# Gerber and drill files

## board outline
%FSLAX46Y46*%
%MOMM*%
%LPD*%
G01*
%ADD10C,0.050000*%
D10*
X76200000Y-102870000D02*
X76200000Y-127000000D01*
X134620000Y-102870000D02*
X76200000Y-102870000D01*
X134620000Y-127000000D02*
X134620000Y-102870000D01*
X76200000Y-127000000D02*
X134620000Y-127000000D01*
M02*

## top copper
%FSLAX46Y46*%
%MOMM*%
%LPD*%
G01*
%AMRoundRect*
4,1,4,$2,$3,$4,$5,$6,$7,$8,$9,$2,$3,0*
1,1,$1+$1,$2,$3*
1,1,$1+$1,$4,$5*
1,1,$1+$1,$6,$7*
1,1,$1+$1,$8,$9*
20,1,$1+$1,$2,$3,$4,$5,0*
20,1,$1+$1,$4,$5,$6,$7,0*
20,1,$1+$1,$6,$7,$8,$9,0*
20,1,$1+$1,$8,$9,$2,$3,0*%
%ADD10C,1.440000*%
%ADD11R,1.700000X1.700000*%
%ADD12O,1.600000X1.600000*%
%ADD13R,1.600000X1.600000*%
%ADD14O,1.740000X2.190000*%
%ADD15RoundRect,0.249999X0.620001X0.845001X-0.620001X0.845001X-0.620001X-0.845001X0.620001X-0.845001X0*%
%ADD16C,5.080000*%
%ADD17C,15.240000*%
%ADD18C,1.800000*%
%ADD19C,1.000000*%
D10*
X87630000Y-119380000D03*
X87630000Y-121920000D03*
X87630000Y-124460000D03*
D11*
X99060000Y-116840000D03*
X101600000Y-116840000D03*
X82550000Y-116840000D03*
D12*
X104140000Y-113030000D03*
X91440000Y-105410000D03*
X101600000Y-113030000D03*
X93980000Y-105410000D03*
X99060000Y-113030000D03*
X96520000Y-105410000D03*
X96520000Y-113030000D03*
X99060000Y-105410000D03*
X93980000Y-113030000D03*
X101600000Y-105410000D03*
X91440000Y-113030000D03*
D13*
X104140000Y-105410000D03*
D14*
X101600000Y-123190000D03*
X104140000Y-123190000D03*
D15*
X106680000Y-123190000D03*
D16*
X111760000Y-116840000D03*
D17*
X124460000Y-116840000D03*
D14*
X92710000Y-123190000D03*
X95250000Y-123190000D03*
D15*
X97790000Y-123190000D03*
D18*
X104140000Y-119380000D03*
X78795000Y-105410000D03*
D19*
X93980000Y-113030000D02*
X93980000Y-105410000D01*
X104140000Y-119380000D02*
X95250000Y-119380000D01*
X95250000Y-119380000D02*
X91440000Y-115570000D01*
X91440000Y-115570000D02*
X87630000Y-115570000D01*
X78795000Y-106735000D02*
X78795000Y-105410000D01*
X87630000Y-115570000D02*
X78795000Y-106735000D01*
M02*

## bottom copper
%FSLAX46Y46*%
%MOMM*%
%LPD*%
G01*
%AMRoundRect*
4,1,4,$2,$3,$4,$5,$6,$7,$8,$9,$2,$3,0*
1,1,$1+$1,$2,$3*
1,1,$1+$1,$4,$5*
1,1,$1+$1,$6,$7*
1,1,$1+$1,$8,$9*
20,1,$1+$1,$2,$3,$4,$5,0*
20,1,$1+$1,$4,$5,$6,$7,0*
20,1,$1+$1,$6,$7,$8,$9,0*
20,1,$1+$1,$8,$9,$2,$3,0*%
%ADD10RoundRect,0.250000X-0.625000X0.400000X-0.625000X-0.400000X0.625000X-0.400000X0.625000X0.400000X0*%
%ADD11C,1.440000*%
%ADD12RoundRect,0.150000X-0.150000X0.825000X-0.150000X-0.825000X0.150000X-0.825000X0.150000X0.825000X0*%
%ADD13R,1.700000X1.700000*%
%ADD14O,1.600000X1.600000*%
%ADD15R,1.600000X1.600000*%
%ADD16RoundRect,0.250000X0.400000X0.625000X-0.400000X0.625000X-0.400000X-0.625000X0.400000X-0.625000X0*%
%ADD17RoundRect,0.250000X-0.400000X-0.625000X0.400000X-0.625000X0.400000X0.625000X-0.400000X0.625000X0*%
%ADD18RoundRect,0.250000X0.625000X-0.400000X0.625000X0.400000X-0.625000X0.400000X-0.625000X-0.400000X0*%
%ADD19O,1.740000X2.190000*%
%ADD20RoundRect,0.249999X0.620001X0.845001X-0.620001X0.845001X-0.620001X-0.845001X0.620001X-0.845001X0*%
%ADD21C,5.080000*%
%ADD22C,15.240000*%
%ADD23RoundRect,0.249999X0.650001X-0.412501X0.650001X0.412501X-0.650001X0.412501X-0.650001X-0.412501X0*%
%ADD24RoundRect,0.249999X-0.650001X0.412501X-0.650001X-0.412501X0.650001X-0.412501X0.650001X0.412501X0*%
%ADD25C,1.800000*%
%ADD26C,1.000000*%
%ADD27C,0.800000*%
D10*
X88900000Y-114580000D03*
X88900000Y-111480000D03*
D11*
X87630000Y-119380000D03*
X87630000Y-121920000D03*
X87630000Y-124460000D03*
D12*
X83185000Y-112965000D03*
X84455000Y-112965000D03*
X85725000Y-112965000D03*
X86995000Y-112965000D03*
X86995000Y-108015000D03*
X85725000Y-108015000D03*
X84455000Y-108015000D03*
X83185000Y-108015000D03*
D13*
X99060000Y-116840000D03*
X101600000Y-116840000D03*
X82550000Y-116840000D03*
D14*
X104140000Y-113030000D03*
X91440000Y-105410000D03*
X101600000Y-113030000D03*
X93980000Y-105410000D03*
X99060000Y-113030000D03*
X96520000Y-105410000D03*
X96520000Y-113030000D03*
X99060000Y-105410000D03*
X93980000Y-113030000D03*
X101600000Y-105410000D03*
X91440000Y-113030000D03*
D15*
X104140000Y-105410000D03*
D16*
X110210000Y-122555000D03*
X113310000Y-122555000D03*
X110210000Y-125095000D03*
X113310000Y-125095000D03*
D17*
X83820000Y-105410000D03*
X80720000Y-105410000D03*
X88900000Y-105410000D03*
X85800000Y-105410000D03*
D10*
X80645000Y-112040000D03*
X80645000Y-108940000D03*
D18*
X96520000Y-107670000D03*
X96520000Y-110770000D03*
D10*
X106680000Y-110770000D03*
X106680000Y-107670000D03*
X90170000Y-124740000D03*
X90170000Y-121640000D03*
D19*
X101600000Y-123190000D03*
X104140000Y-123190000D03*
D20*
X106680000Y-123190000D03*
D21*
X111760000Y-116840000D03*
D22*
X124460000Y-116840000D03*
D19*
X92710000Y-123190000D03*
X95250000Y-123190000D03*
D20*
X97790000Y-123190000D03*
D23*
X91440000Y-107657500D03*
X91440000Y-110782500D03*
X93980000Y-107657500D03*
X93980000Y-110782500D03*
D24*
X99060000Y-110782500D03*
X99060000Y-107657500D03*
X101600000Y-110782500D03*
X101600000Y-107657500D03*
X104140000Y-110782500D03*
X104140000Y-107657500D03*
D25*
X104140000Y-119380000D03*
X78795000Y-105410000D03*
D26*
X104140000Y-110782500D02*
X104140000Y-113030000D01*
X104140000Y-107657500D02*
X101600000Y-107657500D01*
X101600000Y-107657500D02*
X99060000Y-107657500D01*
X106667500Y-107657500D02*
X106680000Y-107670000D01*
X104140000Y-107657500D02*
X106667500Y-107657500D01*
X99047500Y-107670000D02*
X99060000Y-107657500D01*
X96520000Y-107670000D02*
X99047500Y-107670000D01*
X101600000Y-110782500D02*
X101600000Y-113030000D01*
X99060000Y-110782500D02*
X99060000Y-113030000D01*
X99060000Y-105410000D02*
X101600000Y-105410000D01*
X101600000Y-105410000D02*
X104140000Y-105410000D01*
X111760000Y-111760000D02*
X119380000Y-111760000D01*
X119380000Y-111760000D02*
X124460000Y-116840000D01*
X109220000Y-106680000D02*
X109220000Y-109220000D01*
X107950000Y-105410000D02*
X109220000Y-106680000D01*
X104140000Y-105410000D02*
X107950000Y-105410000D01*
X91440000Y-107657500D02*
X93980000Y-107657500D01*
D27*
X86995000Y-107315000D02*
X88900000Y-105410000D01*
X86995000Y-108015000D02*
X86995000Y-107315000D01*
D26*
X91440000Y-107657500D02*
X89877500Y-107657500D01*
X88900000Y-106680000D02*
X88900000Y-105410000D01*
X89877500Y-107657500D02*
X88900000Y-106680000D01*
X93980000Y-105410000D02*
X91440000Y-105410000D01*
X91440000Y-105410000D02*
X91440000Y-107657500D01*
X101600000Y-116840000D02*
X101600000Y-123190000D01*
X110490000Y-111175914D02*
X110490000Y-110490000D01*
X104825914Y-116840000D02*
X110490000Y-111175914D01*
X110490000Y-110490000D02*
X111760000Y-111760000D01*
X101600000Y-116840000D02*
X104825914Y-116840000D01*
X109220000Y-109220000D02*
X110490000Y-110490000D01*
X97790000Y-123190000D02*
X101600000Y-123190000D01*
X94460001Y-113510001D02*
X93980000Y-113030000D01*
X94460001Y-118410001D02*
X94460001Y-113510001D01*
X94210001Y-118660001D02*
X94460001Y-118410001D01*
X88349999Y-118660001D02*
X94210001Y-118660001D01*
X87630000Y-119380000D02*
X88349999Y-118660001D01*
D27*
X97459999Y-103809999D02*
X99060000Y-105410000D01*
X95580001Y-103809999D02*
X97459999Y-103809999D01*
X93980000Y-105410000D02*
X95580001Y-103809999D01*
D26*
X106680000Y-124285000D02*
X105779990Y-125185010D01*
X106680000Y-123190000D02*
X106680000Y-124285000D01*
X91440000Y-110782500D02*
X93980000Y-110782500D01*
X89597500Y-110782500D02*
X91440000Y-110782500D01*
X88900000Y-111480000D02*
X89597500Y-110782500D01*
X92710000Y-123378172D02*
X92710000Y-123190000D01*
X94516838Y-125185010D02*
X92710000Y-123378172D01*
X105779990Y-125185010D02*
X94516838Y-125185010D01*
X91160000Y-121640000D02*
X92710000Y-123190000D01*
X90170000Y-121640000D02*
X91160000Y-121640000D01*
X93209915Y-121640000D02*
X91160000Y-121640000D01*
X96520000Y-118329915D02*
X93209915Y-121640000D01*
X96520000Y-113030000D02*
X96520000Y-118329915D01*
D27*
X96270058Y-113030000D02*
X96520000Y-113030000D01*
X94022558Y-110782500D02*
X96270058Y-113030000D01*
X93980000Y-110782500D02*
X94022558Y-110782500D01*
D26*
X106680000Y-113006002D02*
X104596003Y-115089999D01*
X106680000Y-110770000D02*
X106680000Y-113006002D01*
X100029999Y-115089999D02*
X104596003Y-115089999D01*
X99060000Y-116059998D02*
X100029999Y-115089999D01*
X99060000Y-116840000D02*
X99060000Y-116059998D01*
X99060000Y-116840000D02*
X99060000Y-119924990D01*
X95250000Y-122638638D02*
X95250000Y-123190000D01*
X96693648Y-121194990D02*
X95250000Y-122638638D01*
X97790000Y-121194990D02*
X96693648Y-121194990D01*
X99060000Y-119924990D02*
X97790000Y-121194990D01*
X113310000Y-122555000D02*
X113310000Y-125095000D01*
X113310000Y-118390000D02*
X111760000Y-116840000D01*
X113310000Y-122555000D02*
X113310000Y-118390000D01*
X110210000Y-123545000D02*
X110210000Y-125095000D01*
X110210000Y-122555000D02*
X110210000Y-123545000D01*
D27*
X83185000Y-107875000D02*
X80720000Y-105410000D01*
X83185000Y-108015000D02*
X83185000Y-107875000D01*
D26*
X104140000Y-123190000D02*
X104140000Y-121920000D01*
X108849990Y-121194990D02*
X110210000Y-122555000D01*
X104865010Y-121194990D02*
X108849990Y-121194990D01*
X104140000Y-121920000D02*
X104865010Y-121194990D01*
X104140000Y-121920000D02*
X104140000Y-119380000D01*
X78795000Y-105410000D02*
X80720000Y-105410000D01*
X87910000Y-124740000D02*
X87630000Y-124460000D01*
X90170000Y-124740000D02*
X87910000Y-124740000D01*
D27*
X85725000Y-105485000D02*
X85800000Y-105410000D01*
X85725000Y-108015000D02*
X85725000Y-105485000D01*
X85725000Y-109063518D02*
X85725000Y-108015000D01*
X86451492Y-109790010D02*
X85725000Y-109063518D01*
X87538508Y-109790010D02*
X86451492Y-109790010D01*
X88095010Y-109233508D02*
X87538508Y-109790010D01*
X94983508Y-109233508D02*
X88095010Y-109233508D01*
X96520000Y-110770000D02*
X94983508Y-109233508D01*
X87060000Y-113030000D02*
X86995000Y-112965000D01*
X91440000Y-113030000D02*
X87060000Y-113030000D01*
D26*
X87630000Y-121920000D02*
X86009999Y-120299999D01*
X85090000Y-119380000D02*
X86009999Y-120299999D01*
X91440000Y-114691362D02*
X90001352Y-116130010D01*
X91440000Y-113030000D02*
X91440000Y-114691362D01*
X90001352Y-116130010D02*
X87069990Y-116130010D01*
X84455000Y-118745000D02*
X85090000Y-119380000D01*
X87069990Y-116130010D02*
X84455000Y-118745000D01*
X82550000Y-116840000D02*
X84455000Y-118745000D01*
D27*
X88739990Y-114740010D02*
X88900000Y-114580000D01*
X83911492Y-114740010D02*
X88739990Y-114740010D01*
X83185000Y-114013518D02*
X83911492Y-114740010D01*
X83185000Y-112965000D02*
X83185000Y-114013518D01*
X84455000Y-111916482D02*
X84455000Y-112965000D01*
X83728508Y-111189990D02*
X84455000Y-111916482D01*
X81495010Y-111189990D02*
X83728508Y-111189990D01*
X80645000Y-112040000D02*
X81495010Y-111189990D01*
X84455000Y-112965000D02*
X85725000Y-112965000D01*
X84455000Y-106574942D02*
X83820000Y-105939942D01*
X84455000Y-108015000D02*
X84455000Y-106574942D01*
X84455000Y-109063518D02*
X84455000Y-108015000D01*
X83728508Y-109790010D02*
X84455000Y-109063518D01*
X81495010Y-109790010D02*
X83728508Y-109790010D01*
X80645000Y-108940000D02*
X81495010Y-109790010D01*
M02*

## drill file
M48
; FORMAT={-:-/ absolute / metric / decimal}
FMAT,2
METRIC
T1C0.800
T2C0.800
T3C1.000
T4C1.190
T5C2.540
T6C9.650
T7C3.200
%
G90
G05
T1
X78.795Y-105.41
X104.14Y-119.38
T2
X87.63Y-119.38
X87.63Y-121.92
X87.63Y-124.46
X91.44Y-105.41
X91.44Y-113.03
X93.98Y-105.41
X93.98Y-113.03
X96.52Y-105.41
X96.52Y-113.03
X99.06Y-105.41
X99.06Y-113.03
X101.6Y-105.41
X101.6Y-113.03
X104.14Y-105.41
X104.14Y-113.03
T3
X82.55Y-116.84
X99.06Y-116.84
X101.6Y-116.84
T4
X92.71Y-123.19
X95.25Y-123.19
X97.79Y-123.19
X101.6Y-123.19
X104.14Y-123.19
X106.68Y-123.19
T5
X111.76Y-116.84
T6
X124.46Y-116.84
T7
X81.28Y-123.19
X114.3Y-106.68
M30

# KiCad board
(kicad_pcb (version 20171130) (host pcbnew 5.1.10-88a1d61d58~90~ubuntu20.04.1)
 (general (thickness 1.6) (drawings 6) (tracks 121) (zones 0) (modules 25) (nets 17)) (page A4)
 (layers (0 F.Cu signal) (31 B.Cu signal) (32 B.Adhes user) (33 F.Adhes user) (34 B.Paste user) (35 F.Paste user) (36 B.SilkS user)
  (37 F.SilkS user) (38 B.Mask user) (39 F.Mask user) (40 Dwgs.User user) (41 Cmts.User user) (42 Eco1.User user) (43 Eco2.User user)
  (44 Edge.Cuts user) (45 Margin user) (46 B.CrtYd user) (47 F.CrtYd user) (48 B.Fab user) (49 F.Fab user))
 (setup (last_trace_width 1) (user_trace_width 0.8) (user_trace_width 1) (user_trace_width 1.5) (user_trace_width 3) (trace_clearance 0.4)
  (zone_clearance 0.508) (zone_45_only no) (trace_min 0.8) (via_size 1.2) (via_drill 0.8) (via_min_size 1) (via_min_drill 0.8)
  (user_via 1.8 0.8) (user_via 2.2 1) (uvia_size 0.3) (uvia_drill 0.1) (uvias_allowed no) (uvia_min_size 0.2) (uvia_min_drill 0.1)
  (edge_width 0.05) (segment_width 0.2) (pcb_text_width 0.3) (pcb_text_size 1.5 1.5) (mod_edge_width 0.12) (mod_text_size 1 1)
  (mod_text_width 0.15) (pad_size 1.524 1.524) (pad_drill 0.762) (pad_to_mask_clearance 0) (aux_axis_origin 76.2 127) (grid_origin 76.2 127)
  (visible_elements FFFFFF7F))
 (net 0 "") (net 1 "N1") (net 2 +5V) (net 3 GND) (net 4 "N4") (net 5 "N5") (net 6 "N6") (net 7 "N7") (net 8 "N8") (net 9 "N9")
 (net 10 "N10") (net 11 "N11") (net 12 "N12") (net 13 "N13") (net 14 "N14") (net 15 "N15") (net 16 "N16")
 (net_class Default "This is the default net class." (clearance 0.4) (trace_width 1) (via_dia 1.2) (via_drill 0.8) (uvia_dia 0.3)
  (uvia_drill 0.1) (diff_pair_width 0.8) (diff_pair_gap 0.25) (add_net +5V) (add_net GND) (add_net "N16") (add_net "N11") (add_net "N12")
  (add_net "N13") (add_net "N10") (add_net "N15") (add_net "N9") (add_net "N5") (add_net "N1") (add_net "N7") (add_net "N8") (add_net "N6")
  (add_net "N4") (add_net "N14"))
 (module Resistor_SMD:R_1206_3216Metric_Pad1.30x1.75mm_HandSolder (layer B.Cu) (at 88.9 113.03 270)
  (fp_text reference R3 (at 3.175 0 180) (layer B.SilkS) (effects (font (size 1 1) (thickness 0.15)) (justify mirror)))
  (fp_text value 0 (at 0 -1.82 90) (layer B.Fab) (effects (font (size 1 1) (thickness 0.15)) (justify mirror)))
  (pad 2 smd roundrect (at 1.55 0 270) (size 1.3 1.75) (layers B.Cu B.Paste B.Mask) (roundrect_rratio 0.1923076923076923) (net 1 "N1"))
  (pad 1 smd roundrect (at -1.55 0 270) (size 1.3 1.75) (layers B.Cu B.Paste B.Mask) (roundrect_rratio 0.1923076923076923) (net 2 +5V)))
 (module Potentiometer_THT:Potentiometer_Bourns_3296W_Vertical (layer F.Cu) (at 87.63 124.46 270)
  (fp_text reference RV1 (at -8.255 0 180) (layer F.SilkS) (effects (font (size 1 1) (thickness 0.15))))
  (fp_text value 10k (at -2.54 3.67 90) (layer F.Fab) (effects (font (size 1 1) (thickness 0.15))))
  (pad 3 thru_hole circle (at -5.08 0 270) (size 1.44 1.44) (drill 0.8) (layers *.Cu *.Mask) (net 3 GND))
  (pad 2 thru_hole circle (at -2.54 0 270) (size 1.44 1.44) (drill 0.8) (layers *.Cu *.Mask) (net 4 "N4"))
  (pad 1 thru_hole circle (at 0 0 270) (size 1.44 1.44) (drill 0.8) (layers *.Cu *.Mask) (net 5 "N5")))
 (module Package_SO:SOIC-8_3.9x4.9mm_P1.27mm (layer B.Cu) (at 85.09 110.49 270)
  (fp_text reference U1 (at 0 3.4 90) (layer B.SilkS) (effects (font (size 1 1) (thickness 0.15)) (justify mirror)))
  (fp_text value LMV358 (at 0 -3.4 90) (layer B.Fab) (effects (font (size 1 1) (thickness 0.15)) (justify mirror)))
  (pad 8 smd roundrect (at 2.475 1.905 270) (size 1.95 0.6) (layers B.Cu B.Paste B.Mask) (roundrect_rratio 0.25) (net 1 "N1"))
  (pad 7 smd roundrect (at 2.475 0.635 270) (size 1.95 0.6) (layers B.Cu B.Paste B.Mask) (roundrect_rratio 0.25) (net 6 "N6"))
  (pad 6 smd roundrect (at 2.475 -0.635 270) (size 1.95 0.6) (layers B.Cu B.Paste B.Mask) (roundrect_rratio 0.25) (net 6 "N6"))
  (pad 5 smd roundrect (at 2.475 -1.905 270) (size 1.95 0.6) (layers B.Cu B.Paste B.Mask) (roundrect_rratio 0.25) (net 4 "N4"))
  (pad 4 smd roundrect (at -2.475 -1.905 270) (size 1.95 0.6) (layers B.Cu B.Paste B.Mask) (roundrect_rratio 0.25) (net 3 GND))
  (pad 3 smd roundrect (at -2.475 -0.635 270) (size 1.95 0.6) (layers B.Cu B.Paste B.Mask) (roundrect_rratio 0.25) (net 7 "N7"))
  (pad 2 smd roundrect (at -2.475 0.635 270) (size 1.95 0.6) (layers B.Cu B.Paste B.Mask) (roundrect_rratio 0.25) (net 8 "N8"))
  (pad 1 smd roundrect (at -2.475 1.905 270) (size 1.95 0.6) (layers B.Cu B.Paste B.Mask) (roundrect_rratio 0.25) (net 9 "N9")))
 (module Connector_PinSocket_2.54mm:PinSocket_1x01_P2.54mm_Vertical (layer F.Cu) (at 99.06 116.84)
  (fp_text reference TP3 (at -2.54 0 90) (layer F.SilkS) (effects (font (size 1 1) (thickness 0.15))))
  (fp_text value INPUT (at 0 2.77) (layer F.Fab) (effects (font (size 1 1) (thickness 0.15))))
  (pad 1 thru_hole rect (at 0 0) (size 1.7 1.7) (drill 1) (layers *.Cu *.Mask) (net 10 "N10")))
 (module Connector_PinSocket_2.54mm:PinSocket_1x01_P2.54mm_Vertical (layer F.Cu) (at 101.6 116.84)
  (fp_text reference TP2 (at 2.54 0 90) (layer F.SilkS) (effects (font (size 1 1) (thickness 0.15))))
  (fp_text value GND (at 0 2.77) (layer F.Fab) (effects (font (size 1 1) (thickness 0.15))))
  (pad 1 thru_hole rect (at 0 0) (size 1.7 1.7) (drill 1) (layers *.Cu *.Mask) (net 3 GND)))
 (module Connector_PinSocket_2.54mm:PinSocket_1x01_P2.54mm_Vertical (layer F.Cu) (at 82.55 116.84)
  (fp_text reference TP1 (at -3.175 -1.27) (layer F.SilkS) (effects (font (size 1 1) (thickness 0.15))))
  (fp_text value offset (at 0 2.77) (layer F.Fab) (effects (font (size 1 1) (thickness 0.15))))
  (pad 1 thru_hole rect (at 0 0) (size 1.7 1.7) (drill 1) (layers *.Cu *.Mask) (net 4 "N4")))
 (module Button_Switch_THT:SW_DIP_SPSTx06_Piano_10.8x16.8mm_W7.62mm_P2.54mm (layer F.Cu) (at 104.14 105.41 270)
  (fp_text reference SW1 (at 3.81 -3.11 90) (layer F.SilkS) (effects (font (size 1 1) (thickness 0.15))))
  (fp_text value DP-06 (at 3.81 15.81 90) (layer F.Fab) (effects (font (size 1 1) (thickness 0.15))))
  (pad 12 thru_hole oval (at 7.62 0 270) (size 1.6 1.6) (drill 0.8) (layers *.Cu *.Mask) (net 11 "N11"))
  (pad 6 thru_hole oval (at 0 12.7 270) (size 1.6 1.6) (drill 0.8) (layers *.Cu *.Mask) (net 3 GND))
  (pad 11 thru_hole oval (at 7.62 2.54 270) (size 1.6 1.6) (drill 0.8) (layers *.Cu *.Mask) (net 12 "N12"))
  (pad 5 thru_hole oval (at 0 10.16 270) (size 1.6 1.6) (drill 0.8) (layers *.Cu *.Mask) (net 3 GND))
  (pad 10 thru_hole oval (at 7.62 5.08 270) (size 1.6 1.6) (drill 0.8) (layers *.Cu *.Mask) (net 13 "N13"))
  (pad 4 thru_hole oval (at 0 7.62 270) (size 1.6 1.6) (drill 0.8) (layers *.Cu *.Mask) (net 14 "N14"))
  (pad 9 thru_hole oval (at 7.62 7.62 270) (size 1.6 1.6) (drill 0.8) (layers *.Cu *.Mask) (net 2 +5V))
  (pad 3 thru_hole oval (at 0 5.08 270) (size 1.6 1.6) (drill 0.8) (layers *.Cu *.Mask) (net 3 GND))
  (pad 8 thru_hole oval (at 7.62 10.16 270) (size 1.6 1.6) (drill 0.8) (layers *.Cu *.Mask) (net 3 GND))
  (pad 2 thru_hole oval (at 0 2.54 270) (size 1.6 1.6) (drill 0.8) (layers *.Cu *.Mask) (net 3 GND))
  (pad 7 thru_hole oval (at 7.62 12.7 270) (size 1.6 1.6) (drill 0.8) (layers *.Cu *.Mask) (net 4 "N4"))
  (pad 1 thru_hole rect (at 0 0 270) (size 1.6 1.6) (drill 0.8) (layers *.Cu *.Mask) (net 3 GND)))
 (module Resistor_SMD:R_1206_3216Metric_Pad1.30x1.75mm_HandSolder (layer B.Cu) (at 111.76 122.555 180)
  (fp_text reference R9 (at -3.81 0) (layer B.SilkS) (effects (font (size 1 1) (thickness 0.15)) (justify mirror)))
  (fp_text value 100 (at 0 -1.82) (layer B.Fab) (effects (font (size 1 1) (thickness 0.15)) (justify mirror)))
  (pad 2 smd roundrect (at 1.55 0 180) (size 1.3 1.75) (layers B.Cu B.Paste B.Mask) (roundrect_rratio 0.1923076923076923) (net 9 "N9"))
  (pad 1 smd roundrect (at -1.55 0 180) (size 1.3 1.75) (layers B.Cu B.Paste B.Mask) (roundrect_rratio 0.1923076923076923) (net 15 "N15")))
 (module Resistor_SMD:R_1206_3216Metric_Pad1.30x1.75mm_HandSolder (layer B.Cu) (at 111.76 125.095 180)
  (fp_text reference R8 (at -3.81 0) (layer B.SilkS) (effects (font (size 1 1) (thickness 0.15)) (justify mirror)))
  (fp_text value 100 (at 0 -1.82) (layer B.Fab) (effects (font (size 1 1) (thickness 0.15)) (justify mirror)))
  (pad 2 smd roundrect (at 1.55 0 180) (size 1.3 1.75) (layers B.Cu B.Paste B.Mask) (roundrect_rratio 0.1923076923076923) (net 9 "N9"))
  (pad 1 smd roundrect (at -1.55 0 180) (size 1.3 1.75) (layers B.Cu B.Paste B.Mask) (roundrect_rratio 0.1923076923076923) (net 15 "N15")))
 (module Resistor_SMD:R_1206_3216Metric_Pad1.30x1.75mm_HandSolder (layer B.Cu) (at 82.27 105.41)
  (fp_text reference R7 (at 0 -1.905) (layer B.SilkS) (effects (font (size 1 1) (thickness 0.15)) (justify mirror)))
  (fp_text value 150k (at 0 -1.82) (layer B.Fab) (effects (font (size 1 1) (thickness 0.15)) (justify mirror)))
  (pad 2 smd roundrect (at 1.55 0) (size 1.3 1.75) (layers B.Cu B.Paste B.Mask) (roundrect_rratio 0.1923076923076923) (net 8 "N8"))
  (pad 1 smd roundrect (at -1.55 0) (size 1.3 1.75) (layers B.Cu B.Paste B.Mask) (roundrect_rratio 0.1923076923076923) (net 9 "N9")))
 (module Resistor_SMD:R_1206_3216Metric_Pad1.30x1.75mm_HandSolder (layer B.Cu) (at 87.35 105.41)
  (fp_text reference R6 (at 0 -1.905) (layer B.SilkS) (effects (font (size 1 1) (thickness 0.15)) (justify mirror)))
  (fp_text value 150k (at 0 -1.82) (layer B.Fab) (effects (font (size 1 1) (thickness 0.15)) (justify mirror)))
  (pad 2 smd roundrect (at 1.55 0) (size 1.3 1.75) (layers B.Cu B.Paste B.Mask) (roundrect_rratio 0.1923076923076923) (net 3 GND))
  (pad 1 smd roundrect (at -1.55 0) (size 1.3 1.75) (layers B.Cu B.Paste B.Mask) (roundrect_rratio 0.1923076923076923) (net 7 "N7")))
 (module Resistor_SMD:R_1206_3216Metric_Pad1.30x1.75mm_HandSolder (layer B.Cu) (at 80.645 110.49 270)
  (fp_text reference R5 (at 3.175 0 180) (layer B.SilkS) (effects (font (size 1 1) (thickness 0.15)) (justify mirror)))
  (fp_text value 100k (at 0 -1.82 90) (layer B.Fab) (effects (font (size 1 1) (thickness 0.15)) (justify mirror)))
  (pad 2 smd roundrect (at 1.55 0 270) (size 1.3 1.75) (layers B.Cu B.Paste B.Mask) (roundrect_rratio 0.1923076923076923) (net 6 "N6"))
  (pad 1 smd roundrect (at -1.55 0 270) (size 1.3 1.75) (layers B.Cu B.Paste B.Mask) (roundrect_rratio 0.1923076923076923) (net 8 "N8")))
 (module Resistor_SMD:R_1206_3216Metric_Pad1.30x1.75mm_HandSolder (layer B.Cu) (at 96.52 109.22 90)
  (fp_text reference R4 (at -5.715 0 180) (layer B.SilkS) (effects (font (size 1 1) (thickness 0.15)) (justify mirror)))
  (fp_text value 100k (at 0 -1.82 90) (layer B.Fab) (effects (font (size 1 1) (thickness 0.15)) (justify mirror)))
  (pad 2 smd roundrect (at 1.55 0 90) (size 1.3 1.75) (layers B.Cu B.Paste B.Mask) (roundrect_rratio 0.1923076923076923) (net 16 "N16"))
  (pad 1 smd roundrect (at -1.55 0 90) (size 1.3 1.75) (layers B.Cu B.Paste B.Mask) (roundrect_rratio 0.1923076923076923) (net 7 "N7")))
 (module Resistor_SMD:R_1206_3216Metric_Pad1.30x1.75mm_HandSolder (layer B.Cu) (at 106.68 109.22 270)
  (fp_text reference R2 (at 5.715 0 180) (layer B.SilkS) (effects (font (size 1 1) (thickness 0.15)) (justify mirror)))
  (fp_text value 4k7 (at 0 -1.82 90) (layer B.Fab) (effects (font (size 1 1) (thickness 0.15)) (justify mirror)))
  (pad 2 smd roundrect (at 1.55 0 270) (size 1.3 1.75) (layers B.Cu B.Paste B.Mask) (roundrect_rratio 0.1923076923076923) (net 10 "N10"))
  (pad 1 smd roundrect (at -1.55 0 270) (size 1.3 1.75) (layers B.Cu B.Paste B.Mask) (roundrect_rratio 0.1923076923076923) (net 16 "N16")))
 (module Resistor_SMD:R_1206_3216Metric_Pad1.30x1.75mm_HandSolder (layer B.Cu) (at 90.17 123.19 270)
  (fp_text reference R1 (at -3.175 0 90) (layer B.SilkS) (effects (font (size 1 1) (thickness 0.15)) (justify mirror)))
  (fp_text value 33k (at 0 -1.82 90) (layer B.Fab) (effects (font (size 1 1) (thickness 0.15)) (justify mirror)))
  (pad 2 smd roundrect (at 1.55 0 270) (size 1.3 1.75) (layers B.Cu B.Paste B.Mask) (roundrect_rratio 0.1923076923076923) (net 5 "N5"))
  (pad 1 smd roundrect (at -1.55 0 270) (size 1.3 1.75) (layers B.Cu B.Paste B.Mask) (roundrect_rratio 0.1923076923076923) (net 2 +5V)))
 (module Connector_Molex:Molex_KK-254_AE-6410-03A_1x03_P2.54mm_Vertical (layer F.Cu) (at 106.68 123.19 180)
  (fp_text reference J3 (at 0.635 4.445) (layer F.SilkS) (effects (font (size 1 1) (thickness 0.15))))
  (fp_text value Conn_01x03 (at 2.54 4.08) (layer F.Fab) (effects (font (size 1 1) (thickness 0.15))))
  (pad 3 thru_hole oval (at 5.08 0 180) (size 1.74 2.19) (drill 1.19) (layers *.Cu *.Mask) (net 3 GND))
  (pad 2 thru_hole oval (at 2.54 0 180) (size 1.74 2.19) (drill 1.19) (layers *.Cu *.Mask) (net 9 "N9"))
  (pad 1 thru_hole roundrect (at 0 0 180) (size 1.74 2.19) (drill 1.19) (layers *.Cu *.Mask) (roundrect_rratio 0.1436775862068966)
   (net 2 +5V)))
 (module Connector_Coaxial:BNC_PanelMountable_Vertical (layer F.Cu) (at 111.76 116.84 180)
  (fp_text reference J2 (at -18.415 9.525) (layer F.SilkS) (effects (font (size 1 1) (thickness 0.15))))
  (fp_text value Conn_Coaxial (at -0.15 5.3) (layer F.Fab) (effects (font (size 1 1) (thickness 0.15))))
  (pad 1 thru_hole circle (at 0 0 180) (size 5.08 5.08) (drill 2.54) (layers *.Cu *.Mask) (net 15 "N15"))
  (pad 2 thru_hole circle (at -12.7 0 180) (size 15.24 15.24) (drill 9.65) (layers *.Cu *.Mask) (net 3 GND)))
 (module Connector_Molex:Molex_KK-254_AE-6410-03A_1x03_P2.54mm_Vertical (layer F.Cu) (at 97.79 123.19 180)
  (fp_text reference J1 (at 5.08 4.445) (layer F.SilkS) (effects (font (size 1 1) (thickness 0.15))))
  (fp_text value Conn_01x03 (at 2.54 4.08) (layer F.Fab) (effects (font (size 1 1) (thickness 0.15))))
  (pad 3 thru_hole oval (at 5.08 0 180) (size 1.74 2.19) (drill 1.19) (layers *.Cu *.Mask) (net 2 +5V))
  (pad 2 thru_hole oval (at 2.54 0 180) (size 1.74 2.19) (drill 1.19) (layers *.Cu *.Mask) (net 10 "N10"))
  (pad 1 thru_hole roundrect (at 0 0 180) (size 1.74 2.19) (drill 1.19) (layers *.Cu *.Mask) (roundrect_rratio 0.1436775862068966)
   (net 3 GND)))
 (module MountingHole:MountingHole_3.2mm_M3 (layer F.Cu) (at 114.3 106.68)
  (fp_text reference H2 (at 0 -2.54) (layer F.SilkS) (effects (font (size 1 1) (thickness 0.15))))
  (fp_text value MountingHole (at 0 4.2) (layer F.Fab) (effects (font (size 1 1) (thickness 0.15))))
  (pad 1 np_thru_hole circle (at 0 0) (size 3.2 3.2) (drill 3.2) (layers *.Cu *.Mask)))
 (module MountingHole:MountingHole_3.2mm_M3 (layer F.Cu) (at 81.28 123.19)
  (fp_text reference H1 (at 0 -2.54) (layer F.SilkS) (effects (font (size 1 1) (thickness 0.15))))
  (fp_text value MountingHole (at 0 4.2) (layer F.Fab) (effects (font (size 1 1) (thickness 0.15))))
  (pad 1 np_thru_hole circle (at 0 0) (size 3.2 3.2) (drill 3.2) (layers *.Cu *.Mask)))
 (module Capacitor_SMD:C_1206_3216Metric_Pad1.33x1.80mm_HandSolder (layer B.Cu) (at 91.44 109.22 90)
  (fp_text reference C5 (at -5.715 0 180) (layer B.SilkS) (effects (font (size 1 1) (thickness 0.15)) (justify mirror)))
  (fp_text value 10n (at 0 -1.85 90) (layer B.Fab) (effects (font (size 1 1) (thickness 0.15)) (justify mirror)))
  (pad 2 smd roundrect (at 1.5625 0 90) (size 1.325 1.8) (layers B.Cu B.Paste B.Mask) (roundrect_rratio 0.1886784905660377) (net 3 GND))
  (pad 1 smd roundrect (at -1.5625 0 90) (size 1.325 1.8) (layers B.Cu B.Paste B.Mask) (roundrect_rratio 0.1886784905660377) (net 2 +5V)))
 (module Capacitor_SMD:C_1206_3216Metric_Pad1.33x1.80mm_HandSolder (layer B.Cu) (at 93.98 109.22 90)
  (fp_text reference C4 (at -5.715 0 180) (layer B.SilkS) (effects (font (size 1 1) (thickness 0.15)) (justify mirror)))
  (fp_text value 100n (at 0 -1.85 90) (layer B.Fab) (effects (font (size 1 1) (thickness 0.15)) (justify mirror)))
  (pad 2 smd roundrect (at 1.5625 0 90) (size 1.325 1.8) (layers B.Cu B.Paste B.Mask) (roundrect_rratio 0.1886784905660377) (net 3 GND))
  (pad 1 smd roundrect (at -1.5625 0 90) (size 1.325 1.8) (layers B.Cu B.Paste B.Mask) (roundrect_rratio 0.1886784905660377) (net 2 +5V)))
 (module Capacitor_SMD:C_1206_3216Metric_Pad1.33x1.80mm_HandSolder (layer B.Cu) (at 99.06 109.22 270)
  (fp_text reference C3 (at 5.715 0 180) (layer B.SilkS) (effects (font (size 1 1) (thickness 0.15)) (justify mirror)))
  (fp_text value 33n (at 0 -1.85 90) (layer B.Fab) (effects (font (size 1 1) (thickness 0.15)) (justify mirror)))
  (pad 2 smd roundrect (at 1.5625 0 270) (size 1.325 1.8) (layers B.Cu B.Paste B.Mask) (roundrect_rratio 0.1886784905660377) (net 13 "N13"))
  (pad 1 smd roundrect (at -1.5625 0 270) (size 1.325 1.8) (layers B.Cu B.Paste B.Mask) (roundrect_rratio 0.1886784905660377) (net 16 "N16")))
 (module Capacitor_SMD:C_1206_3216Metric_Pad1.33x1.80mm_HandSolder (layer B.Cu) (at 101.6 109.22 270)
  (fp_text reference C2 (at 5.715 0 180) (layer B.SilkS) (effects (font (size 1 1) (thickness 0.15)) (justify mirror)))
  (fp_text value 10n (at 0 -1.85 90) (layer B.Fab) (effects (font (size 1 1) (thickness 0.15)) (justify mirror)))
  (pad 2 smd roundrect (at 1.5625 0 270) (size 1.325 1.8) (layers B.Cu B.Paste B.Mask) (roundrect_rratio 0.1886784905660377) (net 12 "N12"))
  (pad 1 smd roundrect (at -1.5625 0 270) (size 1.325 1.8) (layers B.Cu B.Paste B.Mask) (roundrect_rratio 0.1886784905660377) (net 16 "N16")))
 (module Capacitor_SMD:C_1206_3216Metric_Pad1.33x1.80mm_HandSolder (layer B.Cu) (at 104.14 109.22 270)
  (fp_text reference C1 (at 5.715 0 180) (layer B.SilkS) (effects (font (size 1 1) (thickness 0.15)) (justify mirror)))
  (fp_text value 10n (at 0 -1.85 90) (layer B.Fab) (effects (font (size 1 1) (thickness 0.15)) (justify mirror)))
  (pad 2 smd roundrect (at 1.5625 0 270) (size 1.325 1.8) (layers B.Cu B.Paste B.Mask) (roundrect_rratio 0.1886784905660377) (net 11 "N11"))
  (pad 1 smd roundrect (at -1.5625 0 270) (size 1.325 1.8) (layers B.Cu B.Paste B.Mask) (roundrect_rratio 0.1886784905660377) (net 16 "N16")))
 (gr_line (start 76.2 102.87) (end 76.2 127) (layer Edge.Cuts) (width 0.05))
 (gr_line (start 134.62 102.87) (end 76.2 102.87) (layer Edge.Cuts) (width 0.05))
 (gr_line (start 134.62 127) (end 134.62 102.87) (layer Edge.Cuts) (width 0.05))
 (gr_line (start 76.2 127) (end 134.62 127) (layer Edge.Cuts) (width 0.05))
 (segment (start 104.14 110.7825) (end 104.14 113.03) (width 1) (layer B.Cu) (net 11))
 (segment (start 104.14 107.6575) (end 101.6 107.6575) (width 1) (layer B.Cu) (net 16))
 (segment (start 101.6 107.6575) (end 99.06 107.6575) (width 1) (layer B.Cu) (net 16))
 (segment (start 106.6675 107.6575) (end 106.68 107.67) (width 1) (layer B.Cu) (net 16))
 (segment (start 104.14 107.6575) (end 106.6675 107.6575) (width 1) (layer B.Cu) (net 16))
 (segment (start 99.0475 107.67) (end 99.06 107.6575) (width 1) (layer B.Cu) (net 16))
 (segment (start 96.52 107.67) (end 99.0475 107.67) (width 1) (layer B.Cu) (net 16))
 (segment (start 101.6 110.7825) (end 101.6 113.03) (width 1) (layer B.Cu) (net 12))
 (segment (start 99.06 110.7825) (end 99.06 113.03) (width 1) (layer B.Cu) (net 13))
 (segment (start 99.06 105.41) (end 101.6 105.41) (width 1) (layer B.Cu) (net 3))
 (segment (start 101.6 105.41) (end 104.14 105.41) (width 1) (layer B.Cu) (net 3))
 (segment (start 111.76 111.76) (end 119.38 111.76) (width 1) (layer B.Cu) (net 3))
 (segment (start 119.38 111.76) (end 124.46 116.84) (width 1) (layer B.Cu) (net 3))
 (segment (start 109.22 106.68) (end 109.22 109.22) (width 1) (layer B.Cu) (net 3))
 (segment (start 107.95 105.41) (end 109.22 106.68) (width 1) (layer B.Cu) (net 3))
 (segment (start 104.14 105.41) (end 107.95 105.41) (width 1) (layer B.Cu) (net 3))
 (segment (start 91.44 107.6575) (end 93.98 107.6575) (width 1) (layer B.Cu) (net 3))
 (segment (start 86.995 107.315) (end 88.9 105.41) (width 0.8) (layer B.Cu) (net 3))
 (segment (start 86.995 108.015) (end 86.995 107.315) (width 0.8) (layer B.Cu) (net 3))
 (segment (start 91.44 107.6575) (end 89.8775 107.6575) (width 1) (layer B.Cu) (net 3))
 (segment (start 88.9 106.68) (end 88.9 105.41) (width 1) (layer B.Cu) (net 3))
 (segment (start 89.8775 107.6575) (end 88.9 106.68) (width 1) (layer B.Cu) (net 3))
 (segment (start 93.98 105.41) (end 91.44 105.41) (width 1) (layer B.Cu) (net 3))
 (segment (start 91.44 105.41) (end 91.44 107.6575) (width 1) (layer B.Cu) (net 3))
 (segment (start 101.6 116.84) (end 101.6 123.19) (width 1) (layer B.Cu) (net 3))
 (segment (start 110.49 111.175914) (end 110.49 110.49) (width 1) (layer B.Cu) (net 3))
 (segment (start 104.825914 116.84) (end 110.49 111.175914) (width 1) (layer B.Cu) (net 3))
 (segment (start 110.49 110.49) (end 111.76 111.76) (width 1) (layer B.Cu) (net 3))
 (segment (start 101.6 116.84) (end 104.825914 116.84) (width 1) (layer B.Cu) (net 3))
 (segment (start 109.22 109.22) (end 110.49 110.49) (width 1) (layer B.Cu) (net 3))
 (segment (start 97.79 123.19) (end 101.6 123.19) (width 1) (layer B.Cu) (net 3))
 (segment (start 93.98 113.03) (end 93.98 105.41) (width 1) (layer F.Cu) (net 3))
 (segment (start 94.460001 113.510001) (end 93.98 113.03) (width 1) (layer B.Cu) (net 3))
 (segment (start 94.460001 118.410001) (end 94.460001 113.510001) (width 1) (layer B.Cu) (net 3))
 (segment (start 94.210001 118.660001) (end 94.460001 118.410001) (width 1) (layer B.Cu) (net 3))
 (segment (start 88.349999 118.660001) (end 94.210001 118.660001) (width 1) (layer B.Cu) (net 3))
 (segment (start 87.63 119.38) (end 88.349999 118.660001) (width 1) (layer B.Cu) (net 3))
 (segment (start 97.459999 103.809999) (end 99.06 105.41) (width 0.8) (layer B.Cu) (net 3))
 (segment (start 95.580001 103.809999) (end 97.459999 103.809999) (width 0.8) (layer B.Cu) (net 3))
 (segment (start 93.98 105.41) (end 95.580001 103.809999) (width 0.8) (layer B.Cu) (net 3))
 (segment (start 106.68 124.285) (end 105.77999 125.18501) (width 1) (layer B.Cu) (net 2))
 (segment (start 106.68 123.19) (end 106.68 124.285) (width 1) (layer B.Cu) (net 2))
 (segment (start 91.44 110.7825) (end 93.98 110.7825) (width 1) (layer B.Cu) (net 2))
 (segment (start 89.5975 110.7825) (end 91.44 110.7825) (width 1) (layer B.Cu) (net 2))
 (segment (start 88.9 111.48) (end 89.5975 110.7825) (width 1) (layer B.Cu) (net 2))
 (segment (start 92.71 123.378172) (end 92.71 123.19) (width 1) (layer B.Cu) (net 2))
 (segment (start 94.516838 125.18501) (end 92.71 123.378172) (width 1) (layer B.Cu) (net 2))
 (segment (start 105.77999 125.18501) (end 94.516838 125.18501) (width 1) (layer B.Cu) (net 2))
 (segment (start 91.16 121.64) (end 92.71 123.19) (width 1) (layer B.Cu) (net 2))
 (segment (start 90.17 121.64) (end 91.16 121.64) (width 1) (layer B.Cu) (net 2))
 (segment (start 93.209915 121.64) (end 91.16 121.64) (width 1) (layer B.Cu) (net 2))
 (segment (start 96.52 118.329915) (end 93.209915 121.64) (width 1) (layer B.Cu) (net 2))
 (segment (start 96.52 113.03) (end 96.52 118.329915) (width 1) (layer B.Cu) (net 2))
 (segment (start 96.270058 113.03) (end 96.52 113.03) (width 0.8) (layer B.Cu) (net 2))
 (segment (start 94.022558 110.7825) (end 96.270058 113.03) (width 0.8) (layer B.Cu) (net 2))
 (segment (start 93.98 110.7825) (end 94.022558 110.7825) (width 0.8) (layer B.Cu) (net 2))
 (segment (start 106.68 113.006002) (end 104.596003 115.089999) (width 1) (layer B.Cu) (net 10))
 (segment (start 106.68 110.77) (end 106.68 113.006002) (width 1) (layer B.Cu) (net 10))
 (segment (start 100.029999 115.089999) (end 104.596003 115.089999) (width 1) (layer B.Cu) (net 10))
 (segment (start 99.06 116.059998) (end 100.029999 115.089999) (width 1) (layer B.Cu) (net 10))
 (segment (start 99.06 116.84) (end 99.06 116.059998) (width 1) (layer B.Cu) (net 10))
 (segment (start 99.06 116.84) (end 99.06 119.92499) (width 1) (layer B.Cu) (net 10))
 (segment (start 95.25 122.638638) (end 95.25 123.19) (width 1) (layer B.Cu) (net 10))
 (segment (start 96.693648 121.19499) (end 95.25 122.638638) (width 1) (layer B.Cu) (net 10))
 (segment (start 97.79 121.19499) (end 96.693648 121.19499) (width 1) (layer B.Cu) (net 10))
 (segment (start 99.06 119.92499) (end 97.79 121.19499) (width 1) (layer B.Cu) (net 10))
 (segment (start 113.31 122.555) (end 113.31 125.095) (width 1) (layer B.Cu) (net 15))
 (segment (start 113.31 118.39) (end 111.76 116.84) (width 1) (layer B.Cu) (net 15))
 (segment (start 113.31 122.555) (end 113.31 118.39) (width 1) (layer B.Cu) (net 15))
 (segment (start 110.21 123.545) (end 110.21 125.095) (width 1) (layer B.Cu) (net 9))
 (segment (start 110.21 122.555) (end 110.21 123.545) (width 1) (layer B.Cu) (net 9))
 (segment (start 83.185 107.875) (end 80.72 105.41) (width 0.8) (layer B.Cu) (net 9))
 (segment (start 83.185 108.015) (end 83.185 107.875) (width 0.8) (layer B.Cu) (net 9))
 (segment (start 104.14 123.19) (end 104.14 121.92) (width 1) (layer B.Cu) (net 9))
 (segment (start 108.84999 121.19499) (end 110.21 122.555) (width 1) (layer B.Cu) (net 9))
 (segment (start 104.86501 121.19499) (end 108.84999 121.19499) (width 1) (layer B.Cu) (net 9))
 (segment (start 104.14 121.92) (end 104.86501 121.19499) (width 1) (layer B.Cu) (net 9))
 (via (at 104.14 119.38) (size 1.8) (drill 0.8) (layers F.Cu B.Cu) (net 9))
 (segment (start 104.14 121.92) (end 104.14 119.38) (width 1) (layer B.Cu) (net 9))
 (segment (start 104.14 119.38) (end 95.25 119.38) (width 1) (layer F.Cu) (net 9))
 (segment (start 95.25 119.38) (end 91.44 115.57) (width 1) (layer F.Cu) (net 9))
 (segment (start 91.44 115.57) (end 87.63 115.57) (width 1) (layer F.Cu) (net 9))
 (via (at 78.795 105.41) (size 1.8) (drill 0.8) (layers F.Cu B.Cu) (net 9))
 (segment (start 78.795 106.735) (end 78.795 105.41) (width 1) (layer F.Cu) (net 9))
 (segment (start 87.63 115.57) (end 78.795 106.735) (width 1) (layer F.Cu) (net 9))
 (segment (start 78.795 105.41) (end 80.72 105.41) (width 1) (layer B.Cu) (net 9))
 (segment (start 87.91 124.74) (end 87.63 124.46) (width 1) (layer B.Cu) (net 5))
 (segment (start 90.17 124.74) (end 87.91 124.74) (width 1) (layer B.Cu) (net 5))
 (segment (start 85.725 105.485) (end 85.8 105.41) (width 0.8) (layer B.Cu) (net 7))
 (segment (start 85.725 108.015) (end 85.725 105.485) (width 0.8) (layer B.Cu) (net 7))
 (segment (start 85.725 109.063518) (end 85.725 108.015) (width 0.8) (layer B.Cu) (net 7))
 (segment (start 86.451492 109.79001) (end 85.725 109.063518) (width 0.8) (layer B.Cu) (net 7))
 (segment (start 87.538508 109.79001) (end 86.451492 109.79001) (width 0.8) (layer B.Cu) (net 7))
 (segment (start 88.09501 109.233508) (end 87.538508 109.79001) (width 0.8) (layer B.Cu) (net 7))
 (segment (start 94.983508 109.233508) (end 88.09501 109.233508) (width 0.8) (layer B.Cu) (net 7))
 (segment (start 96.52 110.77) (end 94.983508 109.233508) (width 0.8) (layer B.Cu) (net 7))
 (segment (start 87.06 113.03) (end 86.995 112.965) (width 0.8) (layer B.Cu) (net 4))
 (segment (start 91.44 113.03) (end 87.06 113.03) (width 0.8) (layer B.Cu) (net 4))
 (segment (start 87.63 121.92) (end 86.009999 120.299999) (width 1) (layer B.Cu) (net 4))
 (segment (start 85.09 119.38) (end 86.009999 120.299999) (width 1) (layer B.Cu) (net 4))
 (segment (start 91.44 114.691362) (end 90.001352 116.13001) (width 1) (layer B.Cu) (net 4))
 (segment (start 91.44 113.03) (end 91.44 114.691362) (width 1) (layer B.Cu) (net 4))
 (segment (start 90.001352 116.13001) (end 87.06999 116.13001) (width 1) (layer B.Cu) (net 4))
 (segment (start 84.455 118.745) (end 85.09 119.38) (width 1) (layer B.Cu) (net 4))
 (segment (start 87.06999 116.13001) (end 84.455 118.745) (width 1) (layer B.Cu) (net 4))
 (segment (start 82.55 116.84) (end 84.455 118.745) (width 1) (layer B.Cu) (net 4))
 (segment (start 88.73999 114.74001) (end 88.9 114.58) (width 0.8) (layer B.Cu) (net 1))
 (segment (start 83.911492 114.74001) (end 88.73999 114.74001) (width 0.8) (layer B.Cu) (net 1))
 (segment (start 83.185 114.013518) (end 83.911492 114.74001) (width 0.8) (layer B.Cu) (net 1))
 (segment (start 83.185 112.965) (end 83.185 114.013518) (width 0.8) (layer B.Cu) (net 1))
 (segment (start 84.455 111.916482) (end 84.455 112.965) (width 0.8) (layer B.Cu) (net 6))
 (segment (start 83.728508 111.18999) (end 84.455 111.916482) (width 0.8) (layer B.Cu) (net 6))
 (segment (start 81.49501 111.18999) (end 83.728508 111.18999) (width 0.8) (layer B.Cu) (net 6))
 (segment (start 80.645 112.04) (end 81.49501 111.18999) (width 0.8) (layer B.Cu) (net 6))
 (segment (start 84.455 112.965) (end 85.725 112.965) (width 0.8) (layer B.Cu) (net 6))
 (segment (start 84.455 106.574942) (end 83.82 105.939942) (width 0.8) (layer B.Cu) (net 8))
 (segment (start 84.455 108.015) (end 84.455 106.574942) (width 0.8) (layer B.Cu) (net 8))
 (segment (start 84.455 109.063518) (end 84.455 108.015) (width 0.8) (layer B.Cu) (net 8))
 (segment (start 83.728508 109.79001) (end 84.455 109.063518) (width 0.8) (layer B.Cu) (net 8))
 (segment (start 81.49501 109.79001) (end 83.728508 109.79001) (width 0.8) (layer B.Cu) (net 8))
 (segment (start 80.645 108.94) (end 81.49501 109.79001) (width 0.8) (layer B.Cu) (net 8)))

